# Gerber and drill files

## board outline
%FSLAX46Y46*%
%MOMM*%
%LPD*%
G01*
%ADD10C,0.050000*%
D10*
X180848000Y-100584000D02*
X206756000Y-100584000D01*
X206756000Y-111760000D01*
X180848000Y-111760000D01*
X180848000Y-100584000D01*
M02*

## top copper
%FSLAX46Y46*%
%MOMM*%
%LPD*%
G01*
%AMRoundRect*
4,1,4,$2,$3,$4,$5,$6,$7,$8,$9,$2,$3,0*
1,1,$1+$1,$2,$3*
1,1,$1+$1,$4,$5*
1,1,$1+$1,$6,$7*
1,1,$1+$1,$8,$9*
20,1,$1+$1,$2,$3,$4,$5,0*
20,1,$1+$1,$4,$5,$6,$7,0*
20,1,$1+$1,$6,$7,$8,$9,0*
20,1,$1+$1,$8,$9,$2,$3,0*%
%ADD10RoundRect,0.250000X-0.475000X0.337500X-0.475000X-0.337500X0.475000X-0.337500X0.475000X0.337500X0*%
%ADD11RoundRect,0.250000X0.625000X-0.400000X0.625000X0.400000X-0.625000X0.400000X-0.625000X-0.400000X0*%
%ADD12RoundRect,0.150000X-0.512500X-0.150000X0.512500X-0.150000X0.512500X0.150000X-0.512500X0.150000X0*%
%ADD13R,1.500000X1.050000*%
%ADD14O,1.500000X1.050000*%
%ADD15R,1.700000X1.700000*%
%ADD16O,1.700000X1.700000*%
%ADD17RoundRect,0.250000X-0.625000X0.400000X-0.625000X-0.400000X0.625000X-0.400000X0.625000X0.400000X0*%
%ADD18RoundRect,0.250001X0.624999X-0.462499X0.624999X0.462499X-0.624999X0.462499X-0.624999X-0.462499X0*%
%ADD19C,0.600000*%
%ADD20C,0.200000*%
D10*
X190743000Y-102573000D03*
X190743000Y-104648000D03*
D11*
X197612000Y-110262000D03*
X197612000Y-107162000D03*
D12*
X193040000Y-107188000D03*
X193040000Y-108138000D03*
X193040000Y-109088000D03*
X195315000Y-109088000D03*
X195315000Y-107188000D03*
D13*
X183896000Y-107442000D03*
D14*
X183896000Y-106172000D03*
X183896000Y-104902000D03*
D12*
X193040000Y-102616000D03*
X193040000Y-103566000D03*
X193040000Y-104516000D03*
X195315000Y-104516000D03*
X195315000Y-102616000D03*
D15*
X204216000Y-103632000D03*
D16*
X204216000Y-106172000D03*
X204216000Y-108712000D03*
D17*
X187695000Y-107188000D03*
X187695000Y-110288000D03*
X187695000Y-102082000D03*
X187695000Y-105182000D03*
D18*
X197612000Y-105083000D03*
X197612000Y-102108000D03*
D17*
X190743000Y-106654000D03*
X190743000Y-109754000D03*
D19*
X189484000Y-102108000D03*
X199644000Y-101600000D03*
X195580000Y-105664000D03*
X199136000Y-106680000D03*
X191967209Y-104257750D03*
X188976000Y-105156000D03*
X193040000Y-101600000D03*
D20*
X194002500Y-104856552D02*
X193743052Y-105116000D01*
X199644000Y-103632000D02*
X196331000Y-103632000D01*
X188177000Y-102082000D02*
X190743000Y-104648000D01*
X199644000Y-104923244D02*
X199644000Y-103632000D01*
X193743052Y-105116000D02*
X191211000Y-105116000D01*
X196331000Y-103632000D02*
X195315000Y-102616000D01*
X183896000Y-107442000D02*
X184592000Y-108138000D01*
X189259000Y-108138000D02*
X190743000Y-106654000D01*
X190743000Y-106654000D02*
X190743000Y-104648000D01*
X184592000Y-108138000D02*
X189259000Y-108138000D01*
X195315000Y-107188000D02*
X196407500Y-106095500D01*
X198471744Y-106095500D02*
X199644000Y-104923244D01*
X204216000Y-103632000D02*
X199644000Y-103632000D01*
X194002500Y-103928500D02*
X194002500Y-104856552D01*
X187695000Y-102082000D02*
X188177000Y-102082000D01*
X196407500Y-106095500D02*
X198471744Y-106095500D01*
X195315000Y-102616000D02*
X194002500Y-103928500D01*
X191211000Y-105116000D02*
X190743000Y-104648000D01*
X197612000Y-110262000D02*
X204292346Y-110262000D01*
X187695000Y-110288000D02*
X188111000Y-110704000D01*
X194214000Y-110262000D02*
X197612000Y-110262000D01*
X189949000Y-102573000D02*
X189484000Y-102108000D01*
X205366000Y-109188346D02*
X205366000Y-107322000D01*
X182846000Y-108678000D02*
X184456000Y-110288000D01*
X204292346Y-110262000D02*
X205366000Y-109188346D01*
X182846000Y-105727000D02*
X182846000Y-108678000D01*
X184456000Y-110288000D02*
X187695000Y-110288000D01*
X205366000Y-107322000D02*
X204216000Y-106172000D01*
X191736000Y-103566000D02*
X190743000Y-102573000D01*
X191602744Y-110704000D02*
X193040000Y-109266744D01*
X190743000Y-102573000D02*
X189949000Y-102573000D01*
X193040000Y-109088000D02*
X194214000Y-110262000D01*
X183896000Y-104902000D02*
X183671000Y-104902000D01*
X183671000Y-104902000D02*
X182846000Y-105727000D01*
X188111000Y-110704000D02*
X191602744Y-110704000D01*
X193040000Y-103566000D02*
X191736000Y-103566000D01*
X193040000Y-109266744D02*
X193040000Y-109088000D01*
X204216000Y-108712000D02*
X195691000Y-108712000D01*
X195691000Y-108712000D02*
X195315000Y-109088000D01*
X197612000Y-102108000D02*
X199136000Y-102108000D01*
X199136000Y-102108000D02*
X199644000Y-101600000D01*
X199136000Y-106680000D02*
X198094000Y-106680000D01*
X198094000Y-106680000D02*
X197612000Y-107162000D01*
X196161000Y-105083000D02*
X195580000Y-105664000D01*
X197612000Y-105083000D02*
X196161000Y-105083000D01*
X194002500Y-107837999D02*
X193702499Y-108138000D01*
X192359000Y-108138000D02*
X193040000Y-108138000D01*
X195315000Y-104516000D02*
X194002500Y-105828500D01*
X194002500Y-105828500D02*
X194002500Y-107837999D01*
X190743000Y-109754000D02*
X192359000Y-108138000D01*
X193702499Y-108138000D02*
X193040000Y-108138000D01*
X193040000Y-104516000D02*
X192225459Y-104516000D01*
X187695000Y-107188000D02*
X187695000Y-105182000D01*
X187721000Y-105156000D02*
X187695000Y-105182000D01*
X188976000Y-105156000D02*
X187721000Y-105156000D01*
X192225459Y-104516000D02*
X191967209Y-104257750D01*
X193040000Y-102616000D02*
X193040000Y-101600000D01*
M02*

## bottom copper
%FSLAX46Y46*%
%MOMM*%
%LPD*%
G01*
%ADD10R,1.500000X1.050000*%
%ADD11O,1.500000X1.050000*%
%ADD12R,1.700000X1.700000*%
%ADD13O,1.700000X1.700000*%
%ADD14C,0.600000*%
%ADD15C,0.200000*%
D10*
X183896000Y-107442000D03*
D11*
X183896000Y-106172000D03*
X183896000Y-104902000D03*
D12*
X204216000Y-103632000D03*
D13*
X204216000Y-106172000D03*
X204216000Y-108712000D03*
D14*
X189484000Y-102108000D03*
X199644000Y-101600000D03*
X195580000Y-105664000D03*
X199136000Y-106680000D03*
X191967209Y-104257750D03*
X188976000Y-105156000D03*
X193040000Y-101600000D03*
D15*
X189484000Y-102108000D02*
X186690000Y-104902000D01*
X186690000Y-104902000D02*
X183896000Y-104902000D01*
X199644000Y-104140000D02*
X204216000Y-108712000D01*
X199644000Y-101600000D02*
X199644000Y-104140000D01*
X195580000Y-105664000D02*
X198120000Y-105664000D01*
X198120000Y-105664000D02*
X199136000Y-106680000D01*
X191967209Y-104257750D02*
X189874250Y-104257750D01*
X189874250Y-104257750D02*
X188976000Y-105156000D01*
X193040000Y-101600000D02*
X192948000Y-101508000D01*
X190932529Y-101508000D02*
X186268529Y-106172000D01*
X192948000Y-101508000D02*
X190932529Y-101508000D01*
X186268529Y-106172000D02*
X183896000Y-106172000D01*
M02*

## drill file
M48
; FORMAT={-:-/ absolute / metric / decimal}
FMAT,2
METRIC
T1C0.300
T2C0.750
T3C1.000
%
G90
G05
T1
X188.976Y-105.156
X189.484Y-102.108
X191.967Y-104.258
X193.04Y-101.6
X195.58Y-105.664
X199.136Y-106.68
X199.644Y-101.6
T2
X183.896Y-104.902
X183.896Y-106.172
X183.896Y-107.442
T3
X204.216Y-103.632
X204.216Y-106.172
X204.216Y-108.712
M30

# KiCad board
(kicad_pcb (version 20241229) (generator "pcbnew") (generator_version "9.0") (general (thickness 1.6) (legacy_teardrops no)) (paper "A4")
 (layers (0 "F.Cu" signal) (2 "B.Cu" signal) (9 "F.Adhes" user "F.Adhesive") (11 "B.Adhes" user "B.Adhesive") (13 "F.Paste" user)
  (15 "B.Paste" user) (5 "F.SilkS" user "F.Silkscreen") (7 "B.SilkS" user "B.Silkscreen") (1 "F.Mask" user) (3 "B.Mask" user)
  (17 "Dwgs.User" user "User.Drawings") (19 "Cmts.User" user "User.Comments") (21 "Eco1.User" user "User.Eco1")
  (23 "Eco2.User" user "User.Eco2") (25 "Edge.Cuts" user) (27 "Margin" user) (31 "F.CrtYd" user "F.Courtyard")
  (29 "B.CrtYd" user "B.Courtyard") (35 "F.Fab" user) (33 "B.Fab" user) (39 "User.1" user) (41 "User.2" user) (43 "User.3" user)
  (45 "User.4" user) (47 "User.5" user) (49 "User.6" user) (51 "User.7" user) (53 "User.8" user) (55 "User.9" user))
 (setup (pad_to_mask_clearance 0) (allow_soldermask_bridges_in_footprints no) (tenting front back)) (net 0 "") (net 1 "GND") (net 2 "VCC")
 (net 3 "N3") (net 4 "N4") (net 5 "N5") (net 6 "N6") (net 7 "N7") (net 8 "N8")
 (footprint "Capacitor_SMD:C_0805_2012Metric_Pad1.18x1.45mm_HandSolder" (layer "F.Cu") (at 190.743 103.6105 -90)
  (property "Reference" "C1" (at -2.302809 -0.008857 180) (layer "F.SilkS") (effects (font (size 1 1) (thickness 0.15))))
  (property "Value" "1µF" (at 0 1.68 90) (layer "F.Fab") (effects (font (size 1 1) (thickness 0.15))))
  (pad "1" smd roundrect (at -1.0375 0 270) (size 1.175 1.45) (layers "F.Cu" "F.Mask" "F.Paste") (roundrect_rratio 0.212766) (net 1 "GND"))
  (pad "2" smd roundrect (at 1.0375 0 270) (size 1.175 1.45) (layers "F.Cu" "F.Mask" "F.Paste") (roundrect_rratio 0.212766) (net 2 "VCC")))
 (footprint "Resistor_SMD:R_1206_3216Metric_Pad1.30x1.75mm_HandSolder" (layer "F.Cu") (at 197.612 108.712 90)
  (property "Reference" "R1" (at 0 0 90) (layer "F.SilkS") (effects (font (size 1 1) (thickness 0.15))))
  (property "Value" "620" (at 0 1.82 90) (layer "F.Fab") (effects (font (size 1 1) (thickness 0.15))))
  (pad "1" smd roundrect (at -1.55 0 90) (size 1.3 1.75) (layers "F.Cu" "F.Mask" "F.Paste") (roundrect_rratio 0.192308) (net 1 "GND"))
  (pad "2" smd roundrect (at 1.55 0 90) (size 1.3 1.75) (layers "F.Cu" "F.Mask" "F.Paste") (roundrect_rratio 0.192308) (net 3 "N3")))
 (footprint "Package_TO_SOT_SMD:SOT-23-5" (layer "F.Cu") (at 194.1775 108.138)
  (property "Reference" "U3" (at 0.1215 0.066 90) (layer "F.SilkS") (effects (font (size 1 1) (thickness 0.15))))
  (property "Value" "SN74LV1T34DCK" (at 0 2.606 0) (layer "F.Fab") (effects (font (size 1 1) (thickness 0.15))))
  (pad "1" smd roundrect (at -1.1375 -0.95) (size 1.325 0.6) (layers "F.Cu" "F.Mask" "F.Paste") (roundrect_rratio 0.25) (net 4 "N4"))
  (pad "2" smd roundrect (at -1.1375 0) (size 1.325 0.6) (layers "F.Cu" "F.Mask" "F.Paste") (roundrect_rratio 0.25) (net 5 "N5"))
  (pad "3" smd roundrect (at -1.1375 0.95) (size 1.325 0.6) (layers "F.Cu" "F.Mask" "F.Paste") (roundrect_rratio 0.25) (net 1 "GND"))
  (pad "4" smd roundrect (at 1.1375 0.95) (size 1.325 0.6) (layers "F.Cu" "F.Mask" "F.Paste") (roundrect_rratio 0.25) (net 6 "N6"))
  (pad "5" smd roundrect (at 1.1375 -0.95) (size 1.325 0.6) (layers "F.Cu" "F.Mask" "F.Paste") (roundrect_rratio 0.25) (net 2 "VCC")))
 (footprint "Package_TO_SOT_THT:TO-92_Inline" (layer "F.Cu") (at 183.896 107.442 90)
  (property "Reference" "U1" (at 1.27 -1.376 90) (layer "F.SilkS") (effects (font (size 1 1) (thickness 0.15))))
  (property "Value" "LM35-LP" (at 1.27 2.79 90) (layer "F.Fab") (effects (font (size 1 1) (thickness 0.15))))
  (pad "1" thru_hole rect (at 0 0 90) (size 1.05 1.5) (drill 0.75) (layers "*.Cu" "*.Mask") (remove_unused_layers no) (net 2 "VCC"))
  (pad "2" thru_hole oval (at 1.27 0 90) (size 1.05 1.5) (drill 0.75) (layers "*.Cu" "*.Mask") (remove_unused_layers no) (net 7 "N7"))
  (pad "3" thru_hole oval (at 2.54 0 90) (size 1.05 1.5) (drill 0.75) (layers "*.Cu" "*.Mask") (remove_unused_layers no) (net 1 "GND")))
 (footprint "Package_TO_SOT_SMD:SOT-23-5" (layer "F.Cu") (at 194.1775 103.566)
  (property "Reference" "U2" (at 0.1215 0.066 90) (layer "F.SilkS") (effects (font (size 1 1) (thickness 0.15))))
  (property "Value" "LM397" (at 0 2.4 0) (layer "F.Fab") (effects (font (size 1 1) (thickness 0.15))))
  (pad "1" smd roundrect (at -1.1375 -0.95) (size 1.325 0.6) (layers "F.Cu" "F.Mask" "F.Paste") (roundrect_rratio 0.25) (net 7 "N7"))
  (pad "2" smd roundrect (at -1.1375 0) (size 1.325 0.6) (layers "F.Cu" "F.Mask" "F.Paste") (roundrect_rratio 0.25) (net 1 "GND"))
  (pad "3" smd roundrect (at -1.1375 0.95) (size 1.325 0.6) (layers "F.Cu" "F.Mask" "F.Paste") (roundrect_rratio 0.25) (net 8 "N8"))
  (pad "4" smd roundrect (at 1.1375 0.95) (size 1.325 0.6) (layers "F.Cu" "F.Mask" "F.Paste") (roundrect_rratio 0.25) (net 5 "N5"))
  (pad "5" smd roundrect (at 1.1375 -0.95) (size 1.325 0.6) (layers "F.Cu" "F.Mask" "F.Paste") (roundrect_rratio 0.25) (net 2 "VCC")))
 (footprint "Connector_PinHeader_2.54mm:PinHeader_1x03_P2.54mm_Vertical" (layer "F.Cu") (at 204.216 103.632)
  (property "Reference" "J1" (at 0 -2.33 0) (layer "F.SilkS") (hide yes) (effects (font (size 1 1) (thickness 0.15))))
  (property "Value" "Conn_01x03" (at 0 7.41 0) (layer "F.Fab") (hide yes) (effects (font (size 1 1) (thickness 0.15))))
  (pad "1" thru_hole rect (at 0 0) (size 1.7 1.7) (drill 1) (layers "*.Cu" "*.Mask") (remove_unused_layers no) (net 2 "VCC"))
  (pad "2" thru_hole oval (at 0 2.54) (size 1.7 1.7) (drill 1) (layers "*.Cu" "*.Mask") (remove_unused_layers no) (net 1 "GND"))
  (pad "3" thru_hole oval (at 0 5.08) (size 1.7 1.7) (drill 1) (layers "*.Cu" "*.Mask") (remove_unused_layers no) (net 6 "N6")))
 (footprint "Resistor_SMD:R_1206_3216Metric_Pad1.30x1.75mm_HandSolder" (layer "F.Cu") (at 187.695 108.738 -90)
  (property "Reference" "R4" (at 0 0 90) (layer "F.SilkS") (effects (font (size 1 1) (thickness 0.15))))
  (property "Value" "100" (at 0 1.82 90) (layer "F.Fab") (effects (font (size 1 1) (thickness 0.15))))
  (pad "1" smd roundrect (at -1.55 0 270) (size 1.3 1.75) (layers "F.Cu" "F.Mask" "F.Paste") (roundrect_rratio 0.192308) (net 8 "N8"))
  (pad "2" smd roundrect (at 1.55 0 270) (size 1.3 1.75) (layers "F.Cu" "F.Mask" "F.Paste") (roundrect_rratio 0.192308) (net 1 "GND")))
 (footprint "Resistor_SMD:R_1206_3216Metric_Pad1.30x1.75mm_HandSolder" (layer "F.Cu") (at 187.695 103.632 -90)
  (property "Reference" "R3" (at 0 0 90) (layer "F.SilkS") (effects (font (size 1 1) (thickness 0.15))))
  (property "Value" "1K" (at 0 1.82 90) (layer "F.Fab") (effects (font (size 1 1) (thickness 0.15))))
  (pad "1" smd roundrect (at -1.55 0 270) (size 1.3 1.75) (layers "F.Cu" "F.Mask" "F.Paste") (roundrect_rratio 0.192308) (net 2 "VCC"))
  (pad "2" smd roundrect (at 1.55 0 270) (size 1.3 1.75) (layers "F.Cu" "F.Mask" "F.Paste") (roundrect_rratio 0.192308) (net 8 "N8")))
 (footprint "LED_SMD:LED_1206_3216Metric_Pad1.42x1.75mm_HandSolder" (layer "F.Cu") (at 197.612 103.5955 90)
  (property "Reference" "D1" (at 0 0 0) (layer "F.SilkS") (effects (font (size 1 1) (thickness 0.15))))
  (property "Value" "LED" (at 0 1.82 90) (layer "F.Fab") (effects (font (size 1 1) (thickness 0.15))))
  (pad "1" smd roundrect (at -1.4875 0 90) (size 1.425 1.75) (layers "F.Cu" "F.Mask" "F.Paste") (roundrect_rratio 0.175439) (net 3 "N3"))
  (pad "2" smd roundrect (at 1.4875 0 90) (size 1.425 1.75) (layers "F.Cu" "F.Mask" "F.Paste") (roundrect_rratio 0.175439) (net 6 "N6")))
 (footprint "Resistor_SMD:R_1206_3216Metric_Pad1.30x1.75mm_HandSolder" (layer "F.Cu") (at 190.743 108.204 -90)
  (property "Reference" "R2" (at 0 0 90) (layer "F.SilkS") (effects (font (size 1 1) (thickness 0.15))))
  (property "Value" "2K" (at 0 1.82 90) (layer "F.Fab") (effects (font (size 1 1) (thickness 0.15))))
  (pad "1" smd roundrect (at -1.55 0 270) (size 1.3 1.75) (layers "F.Cu" "F.Mask" "F.Paste") (roundrect_rratio 0.192308) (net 2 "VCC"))
  (pad "2" smd roundrect (at 1.55 0 270) (size 1.3 1.75) (layers "F.Cu" "F.Mask" "F.Paste") (roundrect_rratio 0.192308) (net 5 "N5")))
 (gr_rect (start 180.848 100.584) (end 206.756 111.76) (stroke (width 0.05) (type default)) (fill no) (layer "Edge.Cuts"))
 (segment (start 194.0025 104.856552) (end 193.743052 105.116) (width 0.2) (layer "F.Cu") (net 2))
 (segment (start 199.644 103.632) (end 196.331 103.632) (width 0.2) (layer "F.Cu") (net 2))
 (segment (start 188.177 102.082) (end 190.743 104.648) (width 0.2) (layer "F.Cu") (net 2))
 (segment (start 199.644 104.923244) (end 199.644 103.632) (width 0.2) (layer "F.Cu") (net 2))
 (segment (start 193.743052 105.116) (end 191.211 105.116) (width 0.2) (layer "F.Cu") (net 2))
 (segment (start 196.331 103.632) (end 195.315 102.616) (width 0.2) (layer "F.Cu") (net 2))
 (segment (start 183.896 107.442) (end 184.592 108.138) (width 0.2) (layer "F.Cu") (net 2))
 (segment (start 189.259 108.138) (end 190.743 106.654) (width 0.2) (layer "F.Cu") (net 2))
 (segment (start 190.743 106.654) (end 190.743 104.648) (width 0.2) (layer "F.Cu") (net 2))
 (segment (start 184.592 108.138) (end 189.259 108.138) (width 0.2) (layer "F.Cu") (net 2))
 (segment (start 195.315 107.188) (end 196.4075 106.0955) (width 0.2) (layer "F.Cu") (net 2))
 (segment (start 198.471744 106.0955) (end 199.644 104.923244) (width 0.2) (layer "F.Cu") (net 2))
 (segment (start 204.216 103.632) (end 199.644 103.632) (width 0.2) (layer "F.Cu") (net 2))
 (segment (start 194.0025 103.9285) (end 194.0025 104.856552) (width 0.2) (layer "F.Cu") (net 2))
 (segment (start 187.695 102.082) (end 188.177 102.082) (width 0.2) (layer "F.Cu") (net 2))
 (segment (start 196.4075 106.0955) (end 198.471744 106.0955) (width 0.2) (layer "F.Cu") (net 2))
 (segment (start 195.315 102.616) (end 194.0025 103.9285) (width 0.2) (layer "F.Cu") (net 2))
 (segment (start 191.211 105.116) (end 190.743 104.648) (width 0.2) (layer "F.Cu") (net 2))
 (segment (start 197.612 110.262) (end 204.292346 110.262) (width 0.2) (layer "F.Cu") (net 1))
 (segment (start 187.695 110.288) (end 188.111 110.704) (width 0.2) (layer "F.Cu") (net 1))
 (segment (start 194.214 110.262) (end 197.612 110.262) (width 0.2) (layer "F.Cu") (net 1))
 (segment (start 189.949 102.573) (end 189.484 102.108) (width 0.2) (layer "F.Cu") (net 1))
 (segment (start 205.366 109.188346) (end 205.366 107.322) (width 0.2) (layer "F.Cu") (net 1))
 (segment (start 182.846 108.678) (end 184.456 110.288) (width 0.2) (layer "F.Cu") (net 1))
 (segment (start 204.292346 110.262) (end 205.366 109.188346) (width 0.2) (layer "F.Cu") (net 1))
 (segment (start 182.846 105.727) (end 182.846 108.678) (width 0.2) (layer "F.Cu") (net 1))
 (segment (start 184.456 110.288) (end 187.695 110.288) (width 0.2) (layer "F.Cu") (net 1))
 (segment (start 205.366 107.322) (end 204.216 106.172) (width 0.2) (layer "F.Cu") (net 1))
 (segment (start 191.736 103.566) (end 190.743 102.573) (width 0.2) (layer "F.Cu") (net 1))
 (segment (start 191.602744 110.704) (end 193.04 109.266744) (width 0.2) (layer "F.Cu") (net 1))
 (segment (start 190.743 102.573) (end 189.949 102.573) (width 0.2) (layer "F.Cu") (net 1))
 (segment (start 193.04 109.088) (end 194.214 110.262) (width 0.2) (layer "F.Cu") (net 1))
 (segment (start 183.896 104.902) (end 183.671 104.902) (width 0.2) (layer "F.Cu") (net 1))
 (segment (start 183.671 104.902) (end 182.846 105.727) (width 0.2) (layer "F.Cu") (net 1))
 (segment (start 188.111 110.704) (end 191.602744 110.704) (width 0.2) (layer "F.Cu") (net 1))
 (segment (start 193.04 103.566) (end 191.736 103.566) (width 0.2) (layer "F.Cu") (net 1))
 (segment (start 193.04 109.266744) (end 193.04 109.088) (width 0.2) (layer "F.Cu") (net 1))
 (via (at 189.484 102.108) (size 0.6) (drill 0.3) (layers "F.Cu" "B.Cu") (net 1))
 (segment (start 189.484 102.108) (end 186.69 104.902) (width 0.2) (layer "B.Cu") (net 1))
 (segment (start 186.69 104.902) (end 183.896 104.902) (width 0.2) (layer "B.Cu") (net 1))
 (segment (start 204.216 108.712) (end 195.691 108.712) (width 0.2) (layer "F.Cu") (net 6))
 (segment (start 195.691 108.712) (end 195.315 109.088) (width 0.2) (layer "F.Cu") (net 6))
 (segment (start 197.612 102.108) (end 199.136 102.108) (width 0.2) (layer "F.Cu") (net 6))
 (segment (start 199.136 102.108) (end 199.644 101.6) (width 0.2) (layer "F.Cu") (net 6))
 (via (at 199.644 101.6) (size 0.6) (drill 0.3) (layers "F.Cu" "B.Cu") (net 6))
 (segment (start 199.644 104.14) (end 204.216 108.712) (width 0.2) (layer "B.Cu") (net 6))
 (segment (start 199.644 101.6) (end 199.644 104.14) (width 0.2) (layer "B.Cu") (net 6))
 (segment (start 199.136 106.68) (end 198.094 106.68) (width 0.2) (layer "F.Cu") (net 3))
 (segment (start 198.094 106.68) (end 197.612 107.162) (width 0.2) (layer "F.Cu") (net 3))
 (segment (start 196.161 105.083) (end 195.58 105.664) (width 0.2) (layer "F.Cu") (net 3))
 (segment (start 197.612 105.083) (end 196.161 105.083) (width 0.2) (layer "F.Cu") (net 3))
 (via (at 195.58 105.664) (size 0.6) (drill 0.3) (layers "F.Cu" "B.Cu") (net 3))
 (via (at 199.136 106.68) (size 0.6) (drill 0.3) (layers "F.Cu" "B.Cu") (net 3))
 (segment (start 195.58 105.664) (end 198.12 105.664) (width 0.2) (layer "B.Cu") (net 3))
 (segment (start 198.12 105.664) (end 199.136 106.68) (width 0.2) (layer "B.Cu") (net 3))
 (segment (start 194.0025 107.837999) (end 193.702499 108.138) (width 0.2) (layer "F.Cu") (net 5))
 (segment (start 192.359 108.138) (end 193.04 108.138) (width 0.2) (layer "F.Cu") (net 5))
 (segment (start 195.315 104.516) (end 194.0025 105.8285) (width 0.2) (layer "F.Cu") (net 5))
 (segment (start 194.0025 105.8285) (end 194.0025 107.837999) (width 0.2) (layer "F.Cu") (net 5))
 (segment (start 190.743 109.754) (end 192.359 108.138) (width 0.2) (layer "F.Cu") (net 5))
 (segment (start 193.702499 108.138) (end 193.04 108.138) (width 0.2) (layer "F.Cu") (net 5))
 (segment (start 193.04 104.516) (end 192.225459 104.516) (width 0.2) (layer "F.Cu") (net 8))
 (segment (start 187.695 107.188) (end 187.695 105.182) (width 0.2) (layer "F.Cu") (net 8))
 (segment (start 187.721 105.156) (end 187.695 105.182) (width 0.2) (layer "F.Cu") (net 8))
 (segment (start 188.976 105.156) (end 187.721 105.156) (width 0.2) (layer "F.Cu") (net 8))
 (segment (start 192.225459 104.516) (end 191.967209 104.25775) (width 0.2) (layer "F.Cu") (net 8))
 (via (at 191.967209 104.25775) (size 0.6) (drill 0.3) (layers "F.Cu" "B.Cu") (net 8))
 (via (at 188.976 105.156) (size 0.6) (drill 0.3) (layers "F.Cu" "B.Cu") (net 8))
 (segment (start 191.967209 104.25775) (end 189.87425 104.25775) (width 0.2) (layer "B.Cu") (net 8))
 (segment (start 189.87425 104.25775) (end 188.976 105.156) (width 0.2) (layer "B.Cu") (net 8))
 (segment (start 193.04 102.616) (end 193.04 101.6) (width 0.2) (layer "F.Cu") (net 7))
 (via (at 193.04 101.6) (size 0.6) (drill 0.3) (layers "F.Cu" "B.Cu") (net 7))
 (segment (start 193.04 101.6) (end 192.948 101.508) (width 0.2) (layer "B.Cu") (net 7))
 (segment (start 190.932529 101.508) (end 186.268529 106.172) (width 0.2) (layer "B.Cu") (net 7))
 (segment (start 192.948 101.508) (end 190.932529 101.508) (width 0.2) (layer "B.Cu") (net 7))
 (segment (start 186.268529 106.172) (end 183.896 106.172) (width 0.2) (layer "B.Cu") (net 7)))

